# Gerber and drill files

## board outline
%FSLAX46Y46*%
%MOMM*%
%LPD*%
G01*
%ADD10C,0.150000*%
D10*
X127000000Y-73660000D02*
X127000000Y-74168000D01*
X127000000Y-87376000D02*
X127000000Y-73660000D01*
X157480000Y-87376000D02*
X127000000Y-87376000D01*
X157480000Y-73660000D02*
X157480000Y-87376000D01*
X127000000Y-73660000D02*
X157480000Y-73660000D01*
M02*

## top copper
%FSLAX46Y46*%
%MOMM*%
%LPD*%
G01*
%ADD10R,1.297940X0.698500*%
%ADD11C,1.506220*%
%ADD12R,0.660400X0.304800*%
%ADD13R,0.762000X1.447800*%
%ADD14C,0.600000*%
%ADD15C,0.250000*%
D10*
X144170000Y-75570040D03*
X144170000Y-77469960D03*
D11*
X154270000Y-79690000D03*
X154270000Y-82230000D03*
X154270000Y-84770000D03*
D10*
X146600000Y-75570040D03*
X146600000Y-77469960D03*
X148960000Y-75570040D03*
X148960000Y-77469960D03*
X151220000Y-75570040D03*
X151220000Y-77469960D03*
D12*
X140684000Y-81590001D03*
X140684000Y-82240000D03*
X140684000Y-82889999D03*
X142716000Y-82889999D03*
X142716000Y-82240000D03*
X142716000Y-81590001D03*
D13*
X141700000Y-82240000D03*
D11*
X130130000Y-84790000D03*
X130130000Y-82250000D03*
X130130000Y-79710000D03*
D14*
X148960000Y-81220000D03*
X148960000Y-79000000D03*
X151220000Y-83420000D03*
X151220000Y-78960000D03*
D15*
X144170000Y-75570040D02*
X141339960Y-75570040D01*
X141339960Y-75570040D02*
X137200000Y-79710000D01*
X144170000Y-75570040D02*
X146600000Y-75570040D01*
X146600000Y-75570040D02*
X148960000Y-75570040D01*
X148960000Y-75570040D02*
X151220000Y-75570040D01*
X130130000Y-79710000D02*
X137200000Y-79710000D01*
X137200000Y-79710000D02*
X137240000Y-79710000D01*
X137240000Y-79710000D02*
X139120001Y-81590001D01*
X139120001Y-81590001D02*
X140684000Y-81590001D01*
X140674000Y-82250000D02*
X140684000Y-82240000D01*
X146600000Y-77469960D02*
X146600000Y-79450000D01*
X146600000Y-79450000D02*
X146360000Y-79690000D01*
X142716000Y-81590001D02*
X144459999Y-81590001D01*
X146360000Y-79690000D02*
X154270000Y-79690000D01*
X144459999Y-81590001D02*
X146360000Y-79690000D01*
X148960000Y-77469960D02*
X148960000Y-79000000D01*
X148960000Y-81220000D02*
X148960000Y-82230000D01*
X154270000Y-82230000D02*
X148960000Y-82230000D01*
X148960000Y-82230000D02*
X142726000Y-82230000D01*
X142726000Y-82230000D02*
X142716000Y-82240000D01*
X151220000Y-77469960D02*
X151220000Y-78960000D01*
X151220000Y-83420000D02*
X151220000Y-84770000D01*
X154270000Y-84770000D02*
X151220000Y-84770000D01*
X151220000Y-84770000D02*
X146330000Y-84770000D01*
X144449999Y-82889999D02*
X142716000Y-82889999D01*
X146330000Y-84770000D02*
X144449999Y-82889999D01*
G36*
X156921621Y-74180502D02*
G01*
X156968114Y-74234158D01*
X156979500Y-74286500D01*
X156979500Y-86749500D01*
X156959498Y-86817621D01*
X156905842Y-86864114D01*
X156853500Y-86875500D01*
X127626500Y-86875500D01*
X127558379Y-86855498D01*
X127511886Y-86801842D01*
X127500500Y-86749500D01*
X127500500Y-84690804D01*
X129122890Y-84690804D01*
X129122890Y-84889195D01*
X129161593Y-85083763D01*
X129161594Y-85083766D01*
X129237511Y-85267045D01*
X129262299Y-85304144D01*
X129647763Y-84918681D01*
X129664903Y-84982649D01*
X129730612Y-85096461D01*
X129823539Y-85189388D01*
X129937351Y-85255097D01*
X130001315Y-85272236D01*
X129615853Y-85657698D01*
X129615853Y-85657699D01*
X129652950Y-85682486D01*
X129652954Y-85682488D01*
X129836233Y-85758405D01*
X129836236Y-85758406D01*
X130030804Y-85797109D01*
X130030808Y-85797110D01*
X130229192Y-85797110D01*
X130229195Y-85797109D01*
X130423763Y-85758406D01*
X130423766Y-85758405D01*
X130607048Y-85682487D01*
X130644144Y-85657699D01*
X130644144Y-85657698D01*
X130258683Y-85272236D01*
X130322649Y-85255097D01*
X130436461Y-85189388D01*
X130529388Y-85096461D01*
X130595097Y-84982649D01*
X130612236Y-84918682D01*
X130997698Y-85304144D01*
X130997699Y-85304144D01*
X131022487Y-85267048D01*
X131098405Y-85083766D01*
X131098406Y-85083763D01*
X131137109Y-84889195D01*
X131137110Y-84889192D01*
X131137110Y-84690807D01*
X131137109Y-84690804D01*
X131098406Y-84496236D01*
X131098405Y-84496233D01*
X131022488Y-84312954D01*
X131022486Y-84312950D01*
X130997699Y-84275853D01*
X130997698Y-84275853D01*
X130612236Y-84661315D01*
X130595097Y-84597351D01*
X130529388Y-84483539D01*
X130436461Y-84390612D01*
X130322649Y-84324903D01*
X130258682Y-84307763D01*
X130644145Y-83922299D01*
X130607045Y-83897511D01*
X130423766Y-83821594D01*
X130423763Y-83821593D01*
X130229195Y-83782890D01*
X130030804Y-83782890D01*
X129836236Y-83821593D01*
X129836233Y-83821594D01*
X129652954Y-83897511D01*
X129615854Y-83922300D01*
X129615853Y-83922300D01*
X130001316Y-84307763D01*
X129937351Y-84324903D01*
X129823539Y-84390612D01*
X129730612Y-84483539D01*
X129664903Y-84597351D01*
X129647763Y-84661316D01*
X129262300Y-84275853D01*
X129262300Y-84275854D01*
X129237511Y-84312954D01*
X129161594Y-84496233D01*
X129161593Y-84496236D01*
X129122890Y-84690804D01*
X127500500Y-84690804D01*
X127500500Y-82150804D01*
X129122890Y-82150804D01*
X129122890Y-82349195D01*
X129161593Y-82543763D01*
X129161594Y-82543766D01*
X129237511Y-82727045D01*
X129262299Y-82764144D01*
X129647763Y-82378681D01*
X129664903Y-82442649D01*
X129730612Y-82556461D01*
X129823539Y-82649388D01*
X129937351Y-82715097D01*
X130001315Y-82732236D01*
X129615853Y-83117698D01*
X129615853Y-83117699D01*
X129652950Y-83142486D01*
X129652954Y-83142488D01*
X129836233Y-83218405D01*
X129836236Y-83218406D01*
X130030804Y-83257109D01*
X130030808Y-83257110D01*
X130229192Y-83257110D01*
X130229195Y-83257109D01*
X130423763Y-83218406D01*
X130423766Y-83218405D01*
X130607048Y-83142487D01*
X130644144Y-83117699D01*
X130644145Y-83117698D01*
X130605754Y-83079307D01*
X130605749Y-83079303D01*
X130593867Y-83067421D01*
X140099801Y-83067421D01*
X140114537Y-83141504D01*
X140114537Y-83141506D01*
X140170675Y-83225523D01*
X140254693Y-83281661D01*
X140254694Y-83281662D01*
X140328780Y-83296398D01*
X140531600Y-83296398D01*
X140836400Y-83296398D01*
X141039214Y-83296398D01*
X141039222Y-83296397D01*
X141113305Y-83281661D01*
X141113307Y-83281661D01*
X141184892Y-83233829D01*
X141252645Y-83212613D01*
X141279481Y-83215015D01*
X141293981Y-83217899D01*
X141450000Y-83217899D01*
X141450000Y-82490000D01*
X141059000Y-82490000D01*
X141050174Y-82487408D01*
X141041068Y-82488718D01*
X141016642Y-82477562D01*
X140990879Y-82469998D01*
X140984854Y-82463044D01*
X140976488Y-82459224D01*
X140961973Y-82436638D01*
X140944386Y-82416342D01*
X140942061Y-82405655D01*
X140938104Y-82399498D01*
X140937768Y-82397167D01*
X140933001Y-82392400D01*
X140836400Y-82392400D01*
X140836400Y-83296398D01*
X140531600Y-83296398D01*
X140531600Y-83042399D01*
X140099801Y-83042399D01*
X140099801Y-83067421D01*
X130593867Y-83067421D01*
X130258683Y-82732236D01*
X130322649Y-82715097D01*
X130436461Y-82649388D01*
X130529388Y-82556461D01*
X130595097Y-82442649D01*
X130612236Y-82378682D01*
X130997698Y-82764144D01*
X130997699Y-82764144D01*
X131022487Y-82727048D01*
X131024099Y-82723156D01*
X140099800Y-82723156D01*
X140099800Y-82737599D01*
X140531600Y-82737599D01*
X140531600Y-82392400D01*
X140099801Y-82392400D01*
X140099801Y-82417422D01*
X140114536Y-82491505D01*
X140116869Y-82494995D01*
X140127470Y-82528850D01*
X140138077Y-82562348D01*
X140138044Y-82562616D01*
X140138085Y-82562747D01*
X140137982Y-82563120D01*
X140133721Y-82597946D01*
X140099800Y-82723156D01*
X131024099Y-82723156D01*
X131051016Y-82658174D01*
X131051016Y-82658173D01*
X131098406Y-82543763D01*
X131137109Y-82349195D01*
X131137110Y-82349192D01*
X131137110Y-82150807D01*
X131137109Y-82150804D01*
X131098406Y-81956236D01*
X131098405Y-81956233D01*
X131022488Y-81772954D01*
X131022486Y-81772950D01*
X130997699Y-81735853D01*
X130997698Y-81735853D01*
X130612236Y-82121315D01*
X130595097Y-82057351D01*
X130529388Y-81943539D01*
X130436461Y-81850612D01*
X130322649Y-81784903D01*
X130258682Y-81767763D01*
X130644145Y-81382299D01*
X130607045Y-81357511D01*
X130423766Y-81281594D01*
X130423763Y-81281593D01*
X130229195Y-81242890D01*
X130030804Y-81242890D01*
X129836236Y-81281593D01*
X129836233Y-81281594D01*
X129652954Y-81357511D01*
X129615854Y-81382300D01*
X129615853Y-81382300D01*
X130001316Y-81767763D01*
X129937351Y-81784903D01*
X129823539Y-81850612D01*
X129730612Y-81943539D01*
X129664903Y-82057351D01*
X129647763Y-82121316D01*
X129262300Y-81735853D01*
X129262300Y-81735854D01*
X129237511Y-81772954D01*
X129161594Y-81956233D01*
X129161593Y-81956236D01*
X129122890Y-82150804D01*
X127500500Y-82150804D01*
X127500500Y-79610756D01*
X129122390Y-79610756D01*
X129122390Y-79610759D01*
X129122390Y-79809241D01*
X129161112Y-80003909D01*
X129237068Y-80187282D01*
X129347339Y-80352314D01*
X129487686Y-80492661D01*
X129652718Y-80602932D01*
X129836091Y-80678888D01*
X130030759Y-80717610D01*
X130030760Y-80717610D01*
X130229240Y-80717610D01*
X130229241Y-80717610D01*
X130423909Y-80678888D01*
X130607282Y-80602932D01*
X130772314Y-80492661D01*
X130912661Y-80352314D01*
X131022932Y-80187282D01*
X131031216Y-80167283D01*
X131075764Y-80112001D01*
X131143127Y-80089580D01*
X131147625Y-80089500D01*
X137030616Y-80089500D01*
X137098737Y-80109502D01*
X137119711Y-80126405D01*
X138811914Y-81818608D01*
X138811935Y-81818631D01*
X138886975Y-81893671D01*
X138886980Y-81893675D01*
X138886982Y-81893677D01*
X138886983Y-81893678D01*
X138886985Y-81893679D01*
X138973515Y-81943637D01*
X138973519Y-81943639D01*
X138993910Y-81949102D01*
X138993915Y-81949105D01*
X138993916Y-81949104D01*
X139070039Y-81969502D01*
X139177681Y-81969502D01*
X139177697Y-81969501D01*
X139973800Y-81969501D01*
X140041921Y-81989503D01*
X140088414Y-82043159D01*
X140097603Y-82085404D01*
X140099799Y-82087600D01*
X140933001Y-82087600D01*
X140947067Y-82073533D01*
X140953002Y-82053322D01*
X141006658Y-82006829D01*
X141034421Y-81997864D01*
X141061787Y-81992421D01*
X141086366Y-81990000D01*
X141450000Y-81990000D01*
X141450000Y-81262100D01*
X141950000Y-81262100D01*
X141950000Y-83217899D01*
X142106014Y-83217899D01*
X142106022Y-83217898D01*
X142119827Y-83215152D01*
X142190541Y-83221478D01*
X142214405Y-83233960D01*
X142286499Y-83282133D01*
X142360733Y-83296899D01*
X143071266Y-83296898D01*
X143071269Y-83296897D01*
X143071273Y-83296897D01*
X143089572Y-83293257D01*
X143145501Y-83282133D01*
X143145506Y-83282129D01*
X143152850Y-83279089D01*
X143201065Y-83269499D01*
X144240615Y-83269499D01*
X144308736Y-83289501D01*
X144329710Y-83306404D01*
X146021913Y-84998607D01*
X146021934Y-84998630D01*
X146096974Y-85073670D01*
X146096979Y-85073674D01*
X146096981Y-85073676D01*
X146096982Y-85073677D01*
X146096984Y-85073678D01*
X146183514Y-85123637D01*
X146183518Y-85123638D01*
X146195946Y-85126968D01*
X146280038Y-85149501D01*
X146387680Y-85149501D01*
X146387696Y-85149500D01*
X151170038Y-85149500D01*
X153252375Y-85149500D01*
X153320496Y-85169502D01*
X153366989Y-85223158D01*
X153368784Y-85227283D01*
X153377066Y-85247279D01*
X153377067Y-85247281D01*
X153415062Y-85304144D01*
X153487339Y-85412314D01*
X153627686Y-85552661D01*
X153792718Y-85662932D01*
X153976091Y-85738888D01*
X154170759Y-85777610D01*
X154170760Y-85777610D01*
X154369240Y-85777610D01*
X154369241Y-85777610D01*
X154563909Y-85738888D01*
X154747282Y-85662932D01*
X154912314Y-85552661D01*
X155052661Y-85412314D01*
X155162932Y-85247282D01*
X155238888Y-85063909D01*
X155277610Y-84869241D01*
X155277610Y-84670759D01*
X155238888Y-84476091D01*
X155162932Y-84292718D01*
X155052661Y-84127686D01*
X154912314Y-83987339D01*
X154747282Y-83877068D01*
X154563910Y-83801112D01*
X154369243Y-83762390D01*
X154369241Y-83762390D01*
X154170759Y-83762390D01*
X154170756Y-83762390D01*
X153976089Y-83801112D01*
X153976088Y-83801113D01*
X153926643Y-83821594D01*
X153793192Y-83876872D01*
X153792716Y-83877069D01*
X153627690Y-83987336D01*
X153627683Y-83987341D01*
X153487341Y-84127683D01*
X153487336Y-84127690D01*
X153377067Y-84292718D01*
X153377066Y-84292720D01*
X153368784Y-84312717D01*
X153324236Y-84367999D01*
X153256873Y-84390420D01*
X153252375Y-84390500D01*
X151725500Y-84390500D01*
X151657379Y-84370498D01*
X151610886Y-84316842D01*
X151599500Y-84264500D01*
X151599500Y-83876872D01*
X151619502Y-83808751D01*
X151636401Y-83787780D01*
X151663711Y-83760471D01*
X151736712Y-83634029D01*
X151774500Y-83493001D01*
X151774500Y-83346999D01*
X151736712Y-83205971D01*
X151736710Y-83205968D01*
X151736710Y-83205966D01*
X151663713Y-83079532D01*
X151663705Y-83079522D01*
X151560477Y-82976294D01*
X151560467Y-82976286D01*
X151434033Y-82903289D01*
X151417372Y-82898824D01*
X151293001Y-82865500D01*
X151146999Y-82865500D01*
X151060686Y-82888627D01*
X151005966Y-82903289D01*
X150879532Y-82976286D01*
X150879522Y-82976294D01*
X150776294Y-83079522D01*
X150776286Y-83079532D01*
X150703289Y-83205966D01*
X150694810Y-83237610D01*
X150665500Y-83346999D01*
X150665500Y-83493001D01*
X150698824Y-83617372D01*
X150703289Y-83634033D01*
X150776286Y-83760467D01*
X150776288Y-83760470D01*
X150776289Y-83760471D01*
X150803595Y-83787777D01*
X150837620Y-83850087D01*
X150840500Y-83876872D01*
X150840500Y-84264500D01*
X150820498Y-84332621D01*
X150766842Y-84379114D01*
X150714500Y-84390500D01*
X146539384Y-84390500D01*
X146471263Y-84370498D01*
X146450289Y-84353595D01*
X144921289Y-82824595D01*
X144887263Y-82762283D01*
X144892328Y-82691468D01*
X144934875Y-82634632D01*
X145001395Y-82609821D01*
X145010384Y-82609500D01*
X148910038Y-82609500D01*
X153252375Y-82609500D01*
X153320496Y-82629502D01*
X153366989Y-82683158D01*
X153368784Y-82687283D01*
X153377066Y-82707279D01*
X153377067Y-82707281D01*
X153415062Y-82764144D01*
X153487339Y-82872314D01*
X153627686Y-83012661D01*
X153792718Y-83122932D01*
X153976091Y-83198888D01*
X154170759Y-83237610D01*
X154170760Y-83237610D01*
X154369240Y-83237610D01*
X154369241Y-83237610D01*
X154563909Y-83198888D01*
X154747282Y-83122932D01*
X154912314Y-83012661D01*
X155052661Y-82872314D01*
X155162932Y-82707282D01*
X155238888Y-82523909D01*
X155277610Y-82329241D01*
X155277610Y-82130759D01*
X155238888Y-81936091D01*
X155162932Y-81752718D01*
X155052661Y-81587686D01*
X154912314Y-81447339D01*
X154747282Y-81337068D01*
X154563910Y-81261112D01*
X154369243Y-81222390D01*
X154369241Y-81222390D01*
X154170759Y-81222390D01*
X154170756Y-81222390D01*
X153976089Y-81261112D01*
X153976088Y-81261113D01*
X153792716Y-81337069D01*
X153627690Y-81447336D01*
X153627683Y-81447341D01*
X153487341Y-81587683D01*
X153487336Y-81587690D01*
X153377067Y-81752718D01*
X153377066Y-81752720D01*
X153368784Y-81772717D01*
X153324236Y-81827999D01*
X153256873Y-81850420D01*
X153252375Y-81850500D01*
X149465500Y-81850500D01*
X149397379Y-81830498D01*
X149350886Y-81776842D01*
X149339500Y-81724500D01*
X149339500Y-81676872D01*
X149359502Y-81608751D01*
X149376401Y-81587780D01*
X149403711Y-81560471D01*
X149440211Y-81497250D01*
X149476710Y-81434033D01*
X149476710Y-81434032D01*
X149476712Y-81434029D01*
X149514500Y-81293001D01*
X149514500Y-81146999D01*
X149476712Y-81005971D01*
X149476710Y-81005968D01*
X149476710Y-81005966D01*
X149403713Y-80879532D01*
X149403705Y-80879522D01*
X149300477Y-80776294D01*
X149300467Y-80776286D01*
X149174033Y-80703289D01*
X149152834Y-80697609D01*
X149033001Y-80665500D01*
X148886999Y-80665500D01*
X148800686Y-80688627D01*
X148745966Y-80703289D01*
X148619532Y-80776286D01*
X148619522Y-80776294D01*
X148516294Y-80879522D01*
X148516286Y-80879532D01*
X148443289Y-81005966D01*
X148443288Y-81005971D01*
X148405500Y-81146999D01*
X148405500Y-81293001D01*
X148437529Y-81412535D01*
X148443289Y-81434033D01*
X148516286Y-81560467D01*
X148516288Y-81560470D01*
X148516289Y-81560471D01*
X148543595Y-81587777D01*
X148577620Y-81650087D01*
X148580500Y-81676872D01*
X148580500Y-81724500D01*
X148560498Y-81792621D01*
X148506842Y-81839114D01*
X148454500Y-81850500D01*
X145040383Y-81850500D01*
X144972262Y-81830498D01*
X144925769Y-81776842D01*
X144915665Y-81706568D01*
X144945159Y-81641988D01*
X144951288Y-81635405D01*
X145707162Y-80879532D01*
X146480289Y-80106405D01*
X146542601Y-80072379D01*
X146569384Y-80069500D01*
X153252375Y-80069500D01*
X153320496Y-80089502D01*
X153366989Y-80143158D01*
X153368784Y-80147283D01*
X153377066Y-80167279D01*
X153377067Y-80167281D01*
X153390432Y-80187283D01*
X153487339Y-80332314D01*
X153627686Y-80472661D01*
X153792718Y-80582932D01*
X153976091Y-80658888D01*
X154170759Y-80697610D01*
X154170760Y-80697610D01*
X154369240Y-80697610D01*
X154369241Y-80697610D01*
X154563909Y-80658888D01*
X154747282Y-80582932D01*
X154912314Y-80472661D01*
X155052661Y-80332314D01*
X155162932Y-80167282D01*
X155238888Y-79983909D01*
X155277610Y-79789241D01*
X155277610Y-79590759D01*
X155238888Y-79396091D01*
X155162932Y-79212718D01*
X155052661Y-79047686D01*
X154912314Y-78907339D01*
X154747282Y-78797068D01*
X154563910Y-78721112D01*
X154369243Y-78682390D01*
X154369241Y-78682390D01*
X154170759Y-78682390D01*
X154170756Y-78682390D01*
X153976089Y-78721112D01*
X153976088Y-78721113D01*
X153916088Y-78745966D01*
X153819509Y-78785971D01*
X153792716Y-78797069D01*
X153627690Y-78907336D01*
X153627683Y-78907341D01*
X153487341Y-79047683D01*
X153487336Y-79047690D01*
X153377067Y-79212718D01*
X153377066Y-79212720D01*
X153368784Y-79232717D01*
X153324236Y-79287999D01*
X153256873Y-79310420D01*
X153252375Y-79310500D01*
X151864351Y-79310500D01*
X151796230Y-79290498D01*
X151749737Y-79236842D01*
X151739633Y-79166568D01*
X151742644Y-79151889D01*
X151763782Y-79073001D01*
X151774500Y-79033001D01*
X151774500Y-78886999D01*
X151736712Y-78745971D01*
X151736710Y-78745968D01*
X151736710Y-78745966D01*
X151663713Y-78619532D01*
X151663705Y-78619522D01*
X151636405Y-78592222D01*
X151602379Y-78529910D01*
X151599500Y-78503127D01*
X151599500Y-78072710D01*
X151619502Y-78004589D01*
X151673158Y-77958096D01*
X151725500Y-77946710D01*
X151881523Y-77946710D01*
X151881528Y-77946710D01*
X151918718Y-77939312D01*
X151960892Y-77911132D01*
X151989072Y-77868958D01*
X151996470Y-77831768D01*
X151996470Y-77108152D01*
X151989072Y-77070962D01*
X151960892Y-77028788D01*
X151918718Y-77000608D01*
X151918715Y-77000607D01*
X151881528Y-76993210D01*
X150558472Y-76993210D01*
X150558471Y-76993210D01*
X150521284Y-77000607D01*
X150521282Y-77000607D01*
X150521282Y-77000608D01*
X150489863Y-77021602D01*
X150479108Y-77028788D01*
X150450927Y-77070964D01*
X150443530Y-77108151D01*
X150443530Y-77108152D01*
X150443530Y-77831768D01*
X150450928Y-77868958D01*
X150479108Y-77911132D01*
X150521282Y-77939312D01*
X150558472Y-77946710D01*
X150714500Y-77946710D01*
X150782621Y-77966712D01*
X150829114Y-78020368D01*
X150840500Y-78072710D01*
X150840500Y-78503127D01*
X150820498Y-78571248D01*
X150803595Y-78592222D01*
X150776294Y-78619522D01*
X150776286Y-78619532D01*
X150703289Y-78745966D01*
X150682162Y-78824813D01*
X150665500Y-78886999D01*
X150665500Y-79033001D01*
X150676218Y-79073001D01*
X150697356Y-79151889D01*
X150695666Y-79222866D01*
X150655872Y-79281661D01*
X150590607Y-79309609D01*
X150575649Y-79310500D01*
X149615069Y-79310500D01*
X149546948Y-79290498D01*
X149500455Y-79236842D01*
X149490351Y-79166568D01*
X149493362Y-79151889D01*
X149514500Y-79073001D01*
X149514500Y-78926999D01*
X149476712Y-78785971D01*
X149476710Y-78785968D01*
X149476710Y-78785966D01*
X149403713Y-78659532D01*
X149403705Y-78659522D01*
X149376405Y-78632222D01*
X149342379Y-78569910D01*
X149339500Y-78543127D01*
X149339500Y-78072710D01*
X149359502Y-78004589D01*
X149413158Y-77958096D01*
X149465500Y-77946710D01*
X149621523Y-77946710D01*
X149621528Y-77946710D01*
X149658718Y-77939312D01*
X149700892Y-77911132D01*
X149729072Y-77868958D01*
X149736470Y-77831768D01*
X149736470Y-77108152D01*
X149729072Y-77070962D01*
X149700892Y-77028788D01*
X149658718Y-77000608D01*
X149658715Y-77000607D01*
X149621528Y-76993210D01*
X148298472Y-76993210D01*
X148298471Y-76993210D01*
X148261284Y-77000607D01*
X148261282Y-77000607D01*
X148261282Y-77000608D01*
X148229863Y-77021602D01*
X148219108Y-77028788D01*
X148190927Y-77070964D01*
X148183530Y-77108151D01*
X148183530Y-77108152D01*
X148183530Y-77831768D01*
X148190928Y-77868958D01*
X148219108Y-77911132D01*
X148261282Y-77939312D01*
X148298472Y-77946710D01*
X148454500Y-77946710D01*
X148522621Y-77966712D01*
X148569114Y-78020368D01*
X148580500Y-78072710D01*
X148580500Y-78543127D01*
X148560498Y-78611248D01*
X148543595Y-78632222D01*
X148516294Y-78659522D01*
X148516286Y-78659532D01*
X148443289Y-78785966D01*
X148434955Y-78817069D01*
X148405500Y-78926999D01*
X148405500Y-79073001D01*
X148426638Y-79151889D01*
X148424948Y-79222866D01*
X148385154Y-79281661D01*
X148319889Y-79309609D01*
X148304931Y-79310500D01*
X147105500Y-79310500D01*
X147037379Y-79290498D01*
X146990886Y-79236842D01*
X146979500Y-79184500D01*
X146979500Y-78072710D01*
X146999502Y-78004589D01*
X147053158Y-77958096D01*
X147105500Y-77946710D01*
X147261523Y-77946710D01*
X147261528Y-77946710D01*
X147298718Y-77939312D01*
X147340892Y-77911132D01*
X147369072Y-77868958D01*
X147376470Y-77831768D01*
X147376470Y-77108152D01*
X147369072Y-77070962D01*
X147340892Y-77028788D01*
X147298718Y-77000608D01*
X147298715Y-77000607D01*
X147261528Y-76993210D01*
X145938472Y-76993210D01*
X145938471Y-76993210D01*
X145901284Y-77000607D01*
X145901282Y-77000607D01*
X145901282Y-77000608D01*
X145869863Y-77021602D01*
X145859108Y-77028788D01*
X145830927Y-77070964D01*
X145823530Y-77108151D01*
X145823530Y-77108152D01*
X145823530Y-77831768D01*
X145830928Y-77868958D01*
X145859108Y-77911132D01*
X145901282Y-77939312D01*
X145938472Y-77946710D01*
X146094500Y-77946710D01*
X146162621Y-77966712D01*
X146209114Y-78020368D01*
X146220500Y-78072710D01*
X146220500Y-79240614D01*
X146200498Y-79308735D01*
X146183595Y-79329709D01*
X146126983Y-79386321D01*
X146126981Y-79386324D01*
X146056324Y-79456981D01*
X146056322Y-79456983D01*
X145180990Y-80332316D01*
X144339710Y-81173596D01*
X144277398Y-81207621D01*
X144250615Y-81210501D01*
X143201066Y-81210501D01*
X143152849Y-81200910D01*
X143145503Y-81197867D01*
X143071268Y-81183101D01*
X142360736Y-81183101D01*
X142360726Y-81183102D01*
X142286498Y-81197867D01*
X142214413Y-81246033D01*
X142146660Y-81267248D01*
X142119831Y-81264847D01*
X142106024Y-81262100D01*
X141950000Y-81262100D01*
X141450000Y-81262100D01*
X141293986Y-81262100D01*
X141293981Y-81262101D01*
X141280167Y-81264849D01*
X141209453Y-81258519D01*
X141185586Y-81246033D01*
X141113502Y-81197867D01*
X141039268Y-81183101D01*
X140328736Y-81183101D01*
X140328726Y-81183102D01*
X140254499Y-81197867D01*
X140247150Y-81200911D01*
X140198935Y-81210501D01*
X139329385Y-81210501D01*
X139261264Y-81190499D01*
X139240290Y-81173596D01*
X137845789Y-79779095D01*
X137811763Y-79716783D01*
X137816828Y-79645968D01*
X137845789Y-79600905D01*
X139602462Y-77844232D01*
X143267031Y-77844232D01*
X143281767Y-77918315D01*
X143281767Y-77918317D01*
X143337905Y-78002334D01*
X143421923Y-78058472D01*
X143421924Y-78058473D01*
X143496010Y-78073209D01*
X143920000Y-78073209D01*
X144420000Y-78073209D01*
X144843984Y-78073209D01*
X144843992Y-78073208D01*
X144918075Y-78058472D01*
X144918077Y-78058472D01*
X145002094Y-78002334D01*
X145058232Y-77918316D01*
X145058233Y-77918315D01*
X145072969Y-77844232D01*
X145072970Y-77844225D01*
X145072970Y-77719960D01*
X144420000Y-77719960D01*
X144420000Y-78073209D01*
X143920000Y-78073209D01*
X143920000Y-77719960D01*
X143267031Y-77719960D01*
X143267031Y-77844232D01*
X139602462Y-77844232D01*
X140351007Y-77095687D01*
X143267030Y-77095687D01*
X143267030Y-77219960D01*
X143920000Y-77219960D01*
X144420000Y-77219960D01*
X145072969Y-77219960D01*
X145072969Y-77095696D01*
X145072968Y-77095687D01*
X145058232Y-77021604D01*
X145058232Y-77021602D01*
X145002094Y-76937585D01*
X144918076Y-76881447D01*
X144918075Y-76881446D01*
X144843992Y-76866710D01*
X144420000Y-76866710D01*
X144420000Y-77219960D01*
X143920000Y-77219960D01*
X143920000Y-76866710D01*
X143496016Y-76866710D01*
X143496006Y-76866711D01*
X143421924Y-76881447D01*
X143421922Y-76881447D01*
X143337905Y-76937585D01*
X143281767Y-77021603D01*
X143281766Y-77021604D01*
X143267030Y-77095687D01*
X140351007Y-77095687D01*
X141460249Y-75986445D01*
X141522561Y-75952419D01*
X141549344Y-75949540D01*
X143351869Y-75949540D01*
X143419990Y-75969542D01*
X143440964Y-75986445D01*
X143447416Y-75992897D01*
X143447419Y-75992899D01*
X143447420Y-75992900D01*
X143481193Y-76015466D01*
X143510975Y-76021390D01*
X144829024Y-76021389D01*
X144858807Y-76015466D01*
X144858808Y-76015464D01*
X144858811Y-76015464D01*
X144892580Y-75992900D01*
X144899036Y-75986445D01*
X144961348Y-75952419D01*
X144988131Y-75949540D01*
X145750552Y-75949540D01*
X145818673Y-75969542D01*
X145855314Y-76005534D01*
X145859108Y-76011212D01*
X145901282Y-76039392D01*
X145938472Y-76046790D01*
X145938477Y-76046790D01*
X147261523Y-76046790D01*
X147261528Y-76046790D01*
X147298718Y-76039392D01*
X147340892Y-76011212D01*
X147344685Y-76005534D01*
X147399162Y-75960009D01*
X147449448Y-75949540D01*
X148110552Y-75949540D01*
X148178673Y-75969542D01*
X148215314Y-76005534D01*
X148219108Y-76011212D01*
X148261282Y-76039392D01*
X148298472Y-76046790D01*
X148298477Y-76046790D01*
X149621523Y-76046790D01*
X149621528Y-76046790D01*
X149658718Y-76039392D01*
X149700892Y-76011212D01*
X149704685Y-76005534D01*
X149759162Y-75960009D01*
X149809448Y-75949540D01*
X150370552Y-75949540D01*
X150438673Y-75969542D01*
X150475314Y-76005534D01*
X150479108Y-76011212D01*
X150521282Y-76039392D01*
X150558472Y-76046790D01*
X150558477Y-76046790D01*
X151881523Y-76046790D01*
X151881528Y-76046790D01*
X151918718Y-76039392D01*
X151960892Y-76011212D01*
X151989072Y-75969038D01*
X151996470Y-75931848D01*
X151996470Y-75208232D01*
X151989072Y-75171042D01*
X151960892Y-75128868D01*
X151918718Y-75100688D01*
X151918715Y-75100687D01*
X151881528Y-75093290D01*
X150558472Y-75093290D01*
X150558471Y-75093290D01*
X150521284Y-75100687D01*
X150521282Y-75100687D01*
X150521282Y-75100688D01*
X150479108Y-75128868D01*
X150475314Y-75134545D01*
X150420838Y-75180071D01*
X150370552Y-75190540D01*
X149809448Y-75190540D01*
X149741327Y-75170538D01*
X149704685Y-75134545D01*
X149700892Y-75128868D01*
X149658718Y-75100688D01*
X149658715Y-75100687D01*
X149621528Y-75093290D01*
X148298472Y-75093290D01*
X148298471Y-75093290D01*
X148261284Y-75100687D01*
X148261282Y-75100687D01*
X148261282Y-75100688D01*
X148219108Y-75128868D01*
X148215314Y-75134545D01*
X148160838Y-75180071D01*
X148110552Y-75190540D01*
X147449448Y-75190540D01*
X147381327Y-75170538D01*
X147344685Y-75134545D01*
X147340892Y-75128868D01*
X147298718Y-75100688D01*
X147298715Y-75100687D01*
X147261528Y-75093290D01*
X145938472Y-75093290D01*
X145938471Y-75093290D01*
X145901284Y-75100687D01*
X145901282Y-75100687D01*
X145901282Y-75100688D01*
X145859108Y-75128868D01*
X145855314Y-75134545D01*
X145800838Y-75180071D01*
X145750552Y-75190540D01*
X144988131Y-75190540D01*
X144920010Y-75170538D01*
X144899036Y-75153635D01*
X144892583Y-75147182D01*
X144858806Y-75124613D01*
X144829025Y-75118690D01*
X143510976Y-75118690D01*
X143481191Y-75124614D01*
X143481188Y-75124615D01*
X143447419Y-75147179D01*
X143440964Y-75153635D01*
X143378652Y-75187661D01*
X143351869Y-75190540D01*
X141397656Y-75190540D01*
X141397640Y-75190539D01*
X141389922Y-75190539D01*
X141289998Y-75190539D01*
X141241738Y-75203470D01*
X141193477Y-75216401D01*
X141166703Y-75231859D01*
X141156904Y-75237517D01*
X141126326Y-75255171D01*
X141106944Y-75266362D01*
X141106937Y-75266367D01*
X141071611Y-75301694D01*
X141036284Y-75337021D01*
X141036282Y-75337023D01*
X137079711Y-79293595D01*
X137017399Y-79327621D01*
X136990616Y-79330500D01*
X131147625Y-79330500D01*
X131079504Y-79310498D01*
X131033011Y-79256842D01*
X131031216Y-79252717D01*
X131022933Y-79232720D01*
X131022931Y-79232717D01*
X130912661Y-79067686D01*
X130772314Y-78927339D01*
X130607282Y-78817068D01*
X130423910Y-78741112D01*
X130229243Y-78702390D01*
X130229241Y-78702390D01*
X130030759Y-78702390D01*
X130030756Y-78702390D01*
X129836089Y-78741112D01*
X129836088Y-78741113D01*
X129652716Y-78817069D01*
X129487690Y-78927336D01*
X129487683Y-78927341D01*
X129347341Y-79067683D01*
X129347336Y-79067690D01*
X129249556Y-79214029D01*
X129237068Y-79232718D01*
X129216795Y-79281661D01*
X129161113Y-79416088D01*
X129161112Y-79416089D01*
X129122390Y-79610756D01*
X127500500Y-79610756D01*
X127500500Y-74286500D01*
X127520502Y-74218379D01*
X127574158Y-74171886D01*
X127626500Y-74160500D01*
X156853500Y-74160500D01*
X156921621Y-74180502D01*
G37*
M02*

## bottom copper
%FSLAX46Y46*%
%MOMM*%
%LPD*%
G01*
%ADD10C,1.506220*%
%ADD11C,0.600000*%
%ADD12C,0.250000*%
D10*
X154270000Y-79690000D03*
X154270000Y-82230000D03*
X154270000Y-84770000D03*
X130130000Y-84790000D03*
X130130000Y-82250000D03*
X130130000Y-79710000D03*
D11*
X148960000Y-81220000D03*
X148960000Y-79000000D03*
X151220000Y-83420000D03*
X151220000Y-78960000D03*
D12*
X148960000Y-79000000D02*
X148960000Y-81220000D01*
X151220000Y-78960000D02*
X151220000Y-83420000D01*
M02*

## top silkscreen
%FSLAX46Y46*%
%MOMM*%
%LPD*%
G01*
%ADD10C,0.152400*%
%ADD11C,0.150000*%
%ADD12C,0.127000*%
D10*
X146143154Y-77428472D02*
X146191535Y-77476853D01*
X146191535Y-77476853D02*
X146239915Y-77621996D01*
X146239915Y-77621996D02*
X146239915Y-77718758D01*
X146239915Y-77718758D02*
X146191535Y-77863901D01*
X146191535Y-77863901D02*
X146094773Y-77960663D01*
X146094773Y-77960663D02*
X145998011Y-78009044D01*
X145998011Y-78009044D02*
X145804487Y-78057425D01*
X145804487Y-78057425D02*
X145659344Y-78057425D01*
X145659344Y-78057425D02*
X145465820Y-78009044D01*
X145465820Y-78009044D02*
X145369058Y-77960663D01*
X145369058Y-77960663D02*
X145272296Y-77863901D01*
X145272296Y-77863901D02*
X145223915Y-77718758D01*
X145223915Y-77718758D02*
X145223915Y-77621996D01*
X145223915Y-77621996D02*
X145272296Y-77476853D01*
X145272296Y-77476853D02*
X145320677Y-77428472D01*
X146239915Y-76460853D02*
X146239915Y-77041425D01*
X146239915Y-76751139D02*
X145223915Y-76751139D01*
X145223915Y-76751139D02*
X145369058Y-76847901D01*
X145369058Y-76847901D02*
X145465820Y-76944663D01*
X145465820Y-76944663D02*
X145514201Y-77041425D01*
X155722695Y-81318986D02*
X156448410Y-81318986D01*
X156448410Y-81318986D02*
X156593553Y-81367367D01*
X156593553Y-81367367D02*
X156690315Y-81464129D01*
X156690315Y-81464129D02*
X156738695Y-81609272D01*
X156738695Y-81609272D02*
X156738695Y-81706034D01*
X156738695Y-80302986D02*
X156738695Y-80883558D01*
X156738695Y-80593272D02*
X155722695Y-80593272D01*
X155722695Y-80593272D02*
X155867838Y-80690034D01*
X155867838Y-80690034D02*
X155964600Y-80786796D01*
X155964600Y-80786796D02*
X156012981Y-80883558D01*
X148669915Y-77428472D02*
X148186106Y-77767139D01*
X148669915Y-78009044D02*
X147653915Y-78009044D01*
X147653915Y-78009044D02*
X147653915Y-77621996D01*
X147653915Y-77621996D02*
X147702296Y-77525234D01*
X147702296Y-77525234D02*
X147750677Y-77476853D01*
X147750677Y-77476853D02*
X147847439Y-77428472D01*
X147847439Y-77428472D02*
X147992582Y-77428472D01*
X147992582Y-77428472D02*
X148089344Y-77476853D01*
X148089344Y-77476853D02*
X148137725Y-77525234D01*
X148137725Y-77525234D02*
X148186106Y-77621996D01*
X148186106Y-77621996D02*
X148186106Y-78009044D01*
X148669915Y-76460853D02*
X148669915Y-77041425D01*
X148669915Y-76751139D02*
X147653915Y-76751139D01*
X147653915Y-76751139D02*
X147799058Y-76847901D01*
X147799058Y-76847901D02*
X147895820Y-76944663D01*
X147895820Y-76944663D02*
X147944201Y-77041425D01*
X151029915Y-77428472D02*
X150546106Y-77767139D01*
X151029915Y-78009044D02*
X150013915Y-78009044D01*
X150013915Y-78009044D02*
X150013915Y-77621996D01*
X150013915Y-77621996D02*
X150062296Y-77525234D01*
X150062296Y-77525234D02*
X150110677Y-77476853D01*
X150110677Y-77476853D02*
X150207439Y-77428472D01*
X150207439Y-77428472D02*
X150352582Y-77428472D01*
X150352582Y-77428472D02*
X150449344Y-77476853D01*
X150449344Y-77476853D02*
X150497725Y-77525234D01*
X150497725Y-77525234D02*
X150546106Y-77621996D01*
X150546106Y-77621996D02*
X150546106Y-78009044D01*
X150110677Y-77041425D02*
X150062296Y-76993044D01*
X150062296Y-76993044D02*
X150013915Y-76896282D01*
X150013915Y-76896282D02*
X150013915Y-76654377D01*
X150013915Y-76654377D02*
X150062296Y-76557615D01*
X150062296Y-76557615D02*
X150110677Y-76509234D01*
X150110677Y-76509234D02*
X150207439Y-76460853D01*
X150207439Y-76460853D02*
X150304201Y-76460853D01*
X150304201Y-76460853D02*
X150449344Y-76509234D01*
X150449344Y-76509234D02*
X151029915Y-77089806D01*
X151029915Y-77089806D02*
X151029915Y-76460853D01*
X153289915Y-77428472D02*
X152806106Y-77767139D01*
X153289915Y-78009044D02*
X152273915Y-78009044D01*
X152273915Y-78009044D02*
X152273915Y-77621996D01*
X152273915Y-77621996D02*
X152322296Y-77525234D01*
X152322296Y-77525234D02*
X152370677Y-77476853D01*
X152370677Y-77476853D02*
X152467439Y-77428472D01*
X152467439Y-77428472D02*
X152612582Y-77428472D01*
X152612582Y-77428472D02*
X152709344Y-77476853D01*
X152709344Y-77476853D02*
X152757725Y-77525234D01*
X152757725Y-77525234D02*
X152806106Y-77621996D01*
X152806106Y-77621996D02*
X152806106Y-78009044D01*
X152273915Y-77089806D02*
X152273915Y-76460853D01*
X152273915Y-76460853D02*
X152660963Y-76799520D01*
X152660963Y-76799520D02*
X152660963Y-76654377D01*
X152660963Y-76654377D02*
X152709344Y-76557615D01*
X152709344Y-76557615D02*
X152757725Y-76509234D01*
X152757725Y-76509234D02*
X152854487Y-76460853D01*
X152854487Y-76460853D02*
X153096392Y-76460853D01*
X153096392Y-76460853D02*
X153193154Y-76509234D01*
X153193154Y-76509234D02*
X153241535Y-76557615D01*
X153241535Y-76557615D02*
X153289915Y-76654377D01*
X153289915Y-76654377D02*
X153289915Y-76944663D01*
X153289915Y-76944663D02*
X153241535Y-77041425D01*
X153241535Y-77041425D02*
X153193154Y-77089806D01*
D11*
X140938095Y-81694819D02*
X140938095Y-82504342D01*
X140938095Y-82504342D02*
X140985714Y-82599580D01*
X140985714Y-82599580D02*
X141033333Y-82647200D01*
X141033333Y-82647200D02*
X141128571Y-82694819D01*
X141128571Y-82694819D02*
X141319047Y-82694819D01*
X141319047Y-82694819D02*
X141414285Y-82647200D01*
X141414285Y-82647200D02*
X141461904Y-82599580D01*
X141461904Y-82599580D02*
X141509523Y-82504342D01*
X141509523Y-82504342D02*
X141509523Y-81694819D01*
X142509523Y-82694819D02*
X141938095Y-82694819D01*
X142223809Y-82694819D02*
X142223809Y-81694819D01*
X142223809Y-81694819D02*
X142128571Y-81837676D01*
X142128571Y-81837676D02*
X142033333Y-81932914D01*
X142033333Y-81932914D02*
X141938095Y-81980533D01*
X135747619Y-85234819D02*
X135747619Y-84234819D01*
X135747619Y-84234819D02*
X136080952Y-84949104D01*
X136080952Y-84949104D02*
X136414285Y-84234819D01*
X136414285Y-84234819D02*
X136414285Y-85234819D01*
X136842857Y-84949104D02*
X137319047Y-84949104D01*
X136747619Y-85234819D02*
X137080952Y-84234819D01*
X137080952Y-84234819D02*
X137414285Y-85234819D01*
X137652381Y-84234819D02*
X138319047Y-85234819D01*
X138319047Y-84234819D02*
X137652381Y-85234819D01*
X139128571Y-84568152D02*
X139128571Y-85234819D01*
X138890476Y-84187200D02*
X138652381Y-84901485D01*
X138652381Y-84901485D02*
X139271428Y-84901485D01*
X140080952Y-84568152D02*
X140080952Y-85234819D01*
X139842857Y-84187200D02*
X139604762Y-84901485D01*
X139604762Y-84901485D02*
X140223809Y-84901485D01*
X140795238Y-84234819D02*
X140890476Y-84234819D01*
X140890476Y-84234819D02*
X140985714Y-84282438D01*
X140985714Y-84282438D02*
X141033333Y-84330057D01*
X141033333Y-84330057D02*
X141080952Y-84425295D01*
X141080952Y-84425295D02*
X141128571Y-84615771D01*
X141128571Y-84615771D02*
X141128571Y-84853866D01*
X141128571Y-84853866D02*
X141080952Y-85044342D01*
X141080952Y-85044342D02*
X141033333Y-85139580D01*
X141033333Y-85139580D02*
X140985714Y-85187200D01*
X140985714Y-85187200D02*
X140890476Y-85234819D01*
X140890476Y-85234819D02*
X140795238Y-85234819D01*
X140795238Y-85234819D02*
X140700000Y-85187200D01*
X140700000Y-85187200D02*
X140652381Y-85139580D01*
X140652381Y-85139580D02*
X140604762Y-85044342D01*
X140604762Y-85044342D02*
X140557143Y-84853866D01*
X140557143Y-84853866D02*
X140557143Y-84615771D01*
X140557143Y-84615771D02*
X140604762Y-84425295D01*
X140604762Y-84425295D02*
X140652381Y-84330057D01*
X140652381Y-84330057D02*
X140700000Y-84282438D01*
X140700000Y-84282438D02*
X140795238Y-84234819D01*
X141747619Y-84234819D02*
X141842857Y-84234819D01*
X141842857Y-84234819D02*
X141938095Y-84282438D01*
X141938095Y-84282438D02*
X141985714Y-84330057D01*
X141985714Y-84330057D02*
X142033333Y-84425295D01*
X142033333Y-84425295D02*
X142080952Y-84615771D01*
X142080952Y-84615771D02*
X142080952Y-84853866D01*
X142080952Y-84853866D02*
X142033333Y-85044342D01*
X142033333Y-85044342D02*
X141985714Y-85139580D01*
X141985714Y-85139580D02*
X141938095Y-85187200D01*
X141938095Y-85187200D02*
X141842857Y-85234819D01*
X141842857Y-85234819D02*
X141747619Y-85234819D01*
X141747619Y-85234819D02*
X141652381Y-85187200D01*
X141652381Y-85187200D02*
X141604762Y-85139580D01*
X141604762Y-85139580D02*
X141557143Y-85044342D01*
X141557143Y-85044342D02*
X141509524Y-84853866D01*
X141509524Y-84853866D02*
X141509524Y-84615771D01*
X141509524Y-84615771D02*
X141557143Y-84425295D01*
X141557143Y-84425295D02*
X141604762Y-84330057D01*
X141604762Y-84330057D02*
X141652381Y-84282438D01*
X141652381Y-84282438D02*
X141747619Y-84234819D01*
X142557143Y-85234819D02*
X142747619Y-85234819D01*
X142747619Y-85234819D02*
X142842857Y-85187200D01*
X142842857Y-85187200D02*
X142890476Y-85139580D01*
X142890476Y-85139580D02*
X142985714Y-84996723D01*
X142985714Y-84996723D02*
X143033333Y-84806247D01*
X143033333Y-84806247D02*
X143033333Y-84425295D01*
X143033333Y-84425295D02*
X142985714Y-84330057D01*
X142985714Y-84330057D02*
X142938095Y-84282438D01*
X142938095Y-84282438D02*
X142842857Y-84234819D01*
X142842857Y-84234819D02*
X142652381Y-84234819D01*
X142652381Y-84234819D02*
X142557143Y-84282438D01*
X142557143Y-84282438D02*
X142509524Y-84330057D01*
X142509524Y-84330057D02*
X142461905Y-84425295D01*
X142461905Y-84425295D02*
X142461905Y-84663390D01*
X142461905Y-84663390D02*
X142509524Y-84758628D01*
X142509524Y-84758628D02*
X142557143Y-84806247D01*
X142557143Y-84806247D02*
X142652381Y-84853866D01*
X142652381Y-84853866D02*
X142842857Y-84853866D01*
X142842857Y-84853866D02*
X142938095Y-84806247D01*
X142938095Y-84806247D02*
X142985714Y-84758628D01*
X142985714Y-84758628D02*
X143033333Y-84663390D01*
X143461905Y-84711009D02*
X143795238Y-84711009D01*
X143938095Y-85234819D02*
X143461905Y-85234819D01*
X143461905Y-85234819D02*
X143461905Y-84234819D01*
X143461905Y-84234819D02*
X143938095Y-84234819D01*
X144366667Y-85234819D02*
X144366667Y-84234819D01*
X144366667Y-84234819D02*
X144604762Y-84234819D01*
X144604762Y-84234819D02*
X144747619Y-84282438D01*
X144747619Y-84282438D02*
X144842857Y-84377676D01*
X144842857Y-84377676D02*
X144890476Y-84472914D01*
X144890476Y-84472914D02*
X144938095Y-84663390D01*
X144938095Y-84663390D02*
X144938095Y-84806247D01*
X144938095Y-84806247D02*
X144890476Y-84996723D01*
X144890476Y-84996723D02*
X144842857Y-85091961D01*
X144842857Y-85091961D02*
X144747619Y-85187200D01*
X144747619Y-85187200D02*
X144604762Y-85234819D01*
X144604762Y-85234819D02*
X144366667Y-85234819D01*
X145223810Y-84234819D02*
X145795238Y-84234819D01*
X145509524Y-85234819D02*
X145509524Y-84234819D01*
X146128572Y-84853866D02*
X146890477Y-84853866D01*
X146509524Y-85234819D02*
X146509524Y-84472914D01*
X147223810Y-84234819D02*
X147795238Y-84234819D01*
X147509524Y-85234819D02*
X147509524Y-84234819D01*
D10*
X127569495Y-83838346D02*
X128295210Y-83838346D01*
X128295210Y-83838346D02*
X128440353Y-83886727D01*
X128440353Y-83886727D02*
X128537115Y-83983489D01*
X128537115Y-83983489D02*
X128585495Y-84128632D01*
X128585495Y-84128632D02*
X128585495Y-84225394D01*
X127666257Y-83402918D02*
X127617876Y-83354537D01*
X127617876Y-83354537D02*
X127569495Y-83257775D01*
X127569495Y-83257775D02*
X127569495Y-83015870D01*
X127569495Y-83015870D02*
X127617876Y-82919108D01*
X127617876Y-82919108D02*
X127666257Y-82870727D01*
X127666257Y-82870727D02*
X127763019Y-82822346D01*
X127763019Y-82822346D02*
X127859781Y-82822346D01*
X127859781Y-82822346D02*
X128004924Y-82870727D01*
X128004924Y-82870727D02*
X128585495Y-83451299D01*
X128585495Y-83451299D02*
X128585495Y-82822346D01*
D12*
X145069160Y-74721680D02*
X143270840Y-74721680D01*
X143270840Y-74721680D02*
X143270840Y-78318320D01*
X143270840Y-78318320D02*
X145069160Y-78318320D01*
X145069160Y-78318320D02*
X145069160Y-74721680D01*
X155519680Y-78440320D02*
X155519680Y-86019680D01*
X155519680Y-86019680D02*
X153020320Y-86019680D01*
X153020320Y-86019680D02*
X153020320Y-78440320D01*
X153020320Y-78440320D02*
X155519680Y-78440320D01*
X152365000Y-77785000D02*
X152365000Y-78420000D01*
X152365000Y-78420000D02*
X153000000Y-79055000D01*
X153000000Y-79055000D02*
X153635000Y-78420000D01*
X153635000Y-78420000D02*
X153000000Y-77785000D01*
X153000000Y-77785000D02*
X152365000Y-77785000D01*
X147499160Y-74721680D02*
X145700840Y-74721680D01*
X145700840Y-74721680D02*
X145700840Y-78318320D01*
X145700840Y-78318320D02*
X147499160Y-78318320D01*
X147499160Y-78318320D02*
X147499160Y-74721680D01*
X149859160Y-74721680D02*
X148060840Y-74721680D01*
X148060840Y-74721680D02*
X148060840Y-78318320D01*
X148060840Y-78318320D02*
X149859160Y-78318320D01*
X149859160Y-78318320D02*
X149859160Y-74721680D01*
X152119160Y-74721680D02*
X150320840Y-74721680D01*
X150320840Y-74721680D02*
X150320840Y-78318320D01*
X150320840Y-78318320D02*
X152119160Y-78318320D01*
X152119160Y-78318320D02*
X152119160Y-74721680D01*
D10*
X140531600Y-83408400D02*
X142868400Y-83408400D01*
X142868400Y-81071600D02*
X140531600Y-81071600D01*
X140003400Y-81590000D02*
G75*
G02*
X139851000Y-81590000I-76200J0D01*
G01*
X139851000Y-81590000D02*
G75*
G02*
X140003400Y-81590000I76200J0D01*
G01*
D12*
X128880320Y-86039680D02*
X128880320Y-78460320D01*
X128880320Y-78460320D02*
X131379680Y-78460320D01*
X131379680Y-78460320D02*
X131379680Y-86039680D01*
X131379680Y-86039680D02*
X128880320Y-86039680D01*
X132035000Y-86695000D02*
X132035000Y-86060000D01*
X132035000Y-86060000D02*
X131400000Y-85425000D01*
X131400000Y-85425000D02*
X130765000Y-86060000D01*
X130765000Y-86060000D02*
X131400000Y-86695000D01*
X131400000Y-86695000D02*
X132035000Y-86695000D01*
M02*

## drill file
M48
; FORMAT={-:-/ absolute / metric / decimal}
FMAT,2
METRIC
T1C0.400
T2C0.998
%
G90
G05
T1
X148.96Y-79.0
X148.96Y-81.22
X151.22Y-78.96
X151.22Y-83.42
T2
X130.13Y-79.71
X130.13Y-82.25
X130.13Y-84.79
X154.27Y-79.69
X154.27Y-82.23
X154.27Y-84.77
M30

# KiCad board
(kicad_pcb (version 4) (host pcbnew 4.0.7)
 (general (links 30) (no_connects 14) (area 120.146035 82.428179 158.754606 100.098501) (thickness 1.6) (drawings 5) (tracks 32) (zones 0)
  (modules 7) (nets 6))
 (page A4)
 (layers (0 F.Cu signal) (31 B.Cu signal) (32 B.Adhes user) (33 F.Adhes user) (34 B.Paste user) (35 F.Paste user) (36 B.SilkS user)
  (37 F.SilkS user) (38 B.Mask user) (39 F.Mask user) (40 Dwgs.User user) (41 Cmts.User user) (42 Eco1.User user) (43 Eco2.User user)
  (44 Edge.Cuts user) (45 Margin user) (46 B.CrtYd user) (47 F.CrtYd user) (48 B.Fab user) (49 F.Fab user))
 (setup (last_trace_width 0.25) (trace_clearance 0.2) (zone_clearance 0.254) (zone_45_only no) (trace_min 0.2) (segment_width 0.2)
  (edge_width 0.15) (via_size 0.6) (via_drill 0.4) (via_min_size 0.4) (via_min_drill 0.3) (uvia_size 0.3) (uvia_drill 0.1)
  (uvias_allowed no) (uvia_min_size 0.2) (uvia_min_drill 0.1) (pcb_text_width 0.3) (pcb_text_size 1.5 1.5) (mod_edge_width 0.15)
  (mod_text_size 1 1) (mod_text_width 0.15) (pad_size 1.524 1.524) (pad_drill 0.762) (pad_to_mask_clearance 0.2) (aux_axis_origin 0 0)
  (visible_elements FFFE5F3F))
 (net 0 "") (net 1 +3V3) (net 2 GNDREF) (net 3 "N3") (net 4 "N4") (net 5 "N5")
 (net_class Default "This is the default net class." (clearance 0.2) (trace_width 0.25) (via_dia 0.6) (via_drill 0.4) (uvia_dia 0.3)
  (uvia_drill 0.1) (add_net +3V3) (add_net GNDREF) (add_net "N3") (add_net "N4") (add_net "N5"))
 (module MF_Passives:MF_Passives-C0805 (layer F.Cu) (at 144.17 76.52 270) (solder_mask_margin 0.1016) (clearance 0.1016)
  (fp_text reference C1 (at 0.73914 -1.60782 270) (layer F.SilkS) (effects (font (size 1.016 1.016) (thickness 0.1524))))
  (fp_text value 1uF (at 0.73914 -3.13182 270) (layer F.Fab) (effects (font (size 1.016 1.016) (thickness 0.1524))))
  (fp_line (start -1.79832 -0.89916) (end -1.79832 0.89916) (layer F.SilkS) (width 0.127))
  (fp_line (start -1.79832 0.89916) (end 1.79832 0.89916) (layer F.SilkS) (width 0.127))
  (fp_line (start 1.79832 0.89916) (end 1.79832 -0.89916) (layer F.SilkS) (width 0.127))
  (fp_line (start 1.79832 -0.89916) (end -1.79832 -0.89916) (layer F.SilkS) (width 0.127))
  (pad 1 smd rect (at -0.94996 0 90) (size 0.6985 1.29794) (layers F.Cu F.Paste F.Mask) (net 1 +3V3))
  (pad 2 smd rect (at 0.94996 0 90) (size 0.6985 1.29794) (layers F.Cu F.Paste F.Mask) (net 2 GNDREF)))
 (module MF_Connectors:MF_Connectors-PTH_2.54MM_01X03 (layer F.Cu) (at 154.27 82.23 270)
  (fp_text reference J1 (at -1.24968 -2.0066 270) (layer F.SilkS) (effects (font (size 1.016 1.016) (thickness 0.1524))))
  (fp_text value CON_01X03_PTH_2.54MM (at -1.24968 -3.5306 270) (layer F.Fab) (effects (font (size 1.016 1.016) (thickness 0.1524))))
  (fp_line (start -3.78968 -1.24968) (end 3.78968 -1.24968) (layer F.SilkS) (width 0.127))
  (fp_line (start 3.78968 -1.24968) (end 3.78968 1.24968) (layer F.SilkS) (width 0.127))
  (fp_line (start 3.78968 1.24968) (end -3.78968 1.24968) (layer F.SilkS) (width 0.127))
  (fp_line (start -3.78968 1.24968) (end -3.78968 -1.24968) (layer F.SilkS) (width 0.127))
  (fp_line (start -4.445 1.905) (end -3.81 1.905) (layer F.SilkS) (width 0.127))
  (fp_line (start -3.81 1.905) (end -3.175 1.27) (layer F.SilkS) (width 0.127))
  (fp_line (start -3.175 1.27) (end -3.81 0.635) (layer F.SilkS) (width 0.127))
  (fp_line (start -3.81 0.635) (end -4.445 1.27) (layer F.SilkS) (width 0.127))
  (fp_line (start -4.445 1.27) (end -4.445 1.905) (layer F.SilkS) (width 0.127))
  (pad 1 thru_hole circle (at -2.54 0 270) (size 1.50622 1.50622) (drill 0.99822) (layers *.Cu *.Mask) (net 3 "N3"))
  (pad 2 thru_hole circle (at 0 0 270) (size 1.50622 1.50622) (drill 0.99822) (layers *.Cu *.Mask) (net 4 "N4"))
  (pad 3 thru_hole circle (at 2.54 0 270) (size 1.50622 1.50622) (drill 0.99822) (layers *.Cu *.Mask) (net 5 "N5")))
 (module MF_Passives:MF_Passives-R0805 (layer F.Cu) (at 146.6 76.52 270) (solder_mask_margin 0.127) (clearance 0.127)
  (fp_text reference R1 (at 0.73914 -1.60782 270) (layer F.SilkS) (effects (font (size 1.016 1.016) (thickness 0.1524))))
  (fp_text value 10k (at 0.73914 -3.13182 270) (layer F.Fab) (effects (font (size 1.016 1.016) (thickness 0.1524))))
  (fp_line (start -1.79832 -0.89916) (end -1.79832 0.89916) (layer F.SilkS) (width 0.127))
  (fp_line (start -1.79832 0.89916) (end 1.79832 0.89916) (layer F.SilkS) (width 0.127))
  (fp_line (start 1.79832 0.89916) (end 1.79832 -0.89916) (layer F.SilkS) (width 0.127))
  (fp_line (start 1.79832 -0.89916) (end -1.79832 -0.89916) (layer F.SilkS) (width 0.127))
  (pad 1 smd rect (at -0.94996 0 90) (size 0.6985 1.29794) (layers F.Cu F.Paste F.Mask) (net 1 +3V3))
  (pad 2 smd rect (at 0.94996 0 90) (size 0.6985 1.29794) (layers F.Cu F.Paste F.Mask) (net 3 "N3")))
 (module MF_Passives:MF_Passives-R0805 (layer F.Cu) (at 148.96 76.52 270) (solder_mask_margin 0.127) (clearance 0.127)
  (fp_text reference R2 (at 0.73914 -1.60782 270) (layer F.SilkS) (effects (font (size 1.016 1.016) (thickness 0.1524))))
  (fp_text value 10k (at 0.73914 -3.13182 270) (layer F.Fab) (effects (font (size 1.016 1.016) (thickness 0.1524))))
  (fp_line (start -1.79832 -0.89916) (end -1.79832 0.89916) (layer F.SilkS) (width 0.127))
  (fp_line (start -1.79832 0.89916) (end 1.79832 0.89916) (layer F.SilkS) (width 0.127))
  (fp_line (start 1.79832 0.89916) (end 1.79832 -0.89916) (layer F.SilkS) (width 0.127))
  (fp_line (start 1.79832 -0.89916) (end -1.79832 -0.89916) (layer F.SilkS) (width 0.127))
  (pad 1 smd rect (at -0.94996 0 90) (size 0.6985 1.29794) (layers F.Cu F.Paste F.Mask) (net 1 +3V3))
  (pad 2 smd rect (at 0.94996 0 90) (size 0.6985 1.29794) (layers F.Cu F.Paste F.Mask) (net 4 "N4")))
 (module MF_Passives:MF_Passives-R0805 (layer F.Cu) (at 151.22 76.52 270) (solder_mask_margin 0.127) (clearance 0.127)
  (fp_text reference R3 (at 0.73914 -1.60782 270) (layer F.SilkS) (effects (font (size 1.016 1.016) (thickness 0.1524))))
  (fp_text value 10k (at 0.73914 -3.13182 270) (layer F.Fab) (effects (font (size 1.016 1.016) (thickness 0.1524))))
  (fp_line (start -1.79832 -0.89916) (end -1.79832 0.89916) (layer F.SilkS) (width 0.127))
  (fp_line (start -1.79832 0.89916) (end 1.79832 0.89916) (layer F.SilkS) (width 0.127))
  (fp_line (start 1.79832 0.89916) (end 1.79832 -0.89916) (layer F.SilkS) (width 0.127))
  (fp_line (start 1.79832 -0.89916) (end -1.79832 -0.89916) (layer F.SilkS) (width 0.127))
  (pad 1 smd rect (at -0.94996 0 90) (size 0.6985 1.29794) (layers F.Cu F.Paste F.Mask) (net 1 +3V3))
  (pad 2 smd rect (at 0.94996 0 90) (size 0.6985 1.29794) (layers F.Cu F.Paste F.Mask) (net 5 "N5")))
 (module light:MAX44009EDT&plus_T (layer F.Cu) (at 141.7 82.24)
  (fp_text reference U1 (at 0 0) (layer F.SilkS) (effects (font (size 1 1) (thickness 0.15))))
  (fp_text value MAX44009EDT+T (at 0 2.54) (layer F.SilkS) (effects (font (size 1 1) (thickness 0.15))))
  (fp_line (start -1.1684 1.1684) (end 1.1684 1.1684) (layer F.SilkS) (width 0.1524))
  (fp_line (start 1.1684 -1.1684) (end -1.1684 -1.1684) (layer F.SilkS) (width 0.1524))
  (fp_circle (center -1.7728 -0.65) (end -1.6966 -0.65) (layer F.SilkS) (width 0.1524))
  (pad 1 smd rect (at -1.016 -0.649999) (size 0.6604 0.3048) (layers F.Cu) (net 1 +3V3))
  (pad 1 smd rect (at -1.016 -0.649999) (size 0.6604 0.3048) (layers F.Paste) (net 1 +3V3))
  (pad 1 smd rect (at -1.016 -0.649999) (size 0.6604 0.3048) (layers F.Mask) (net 1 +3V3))
  (pad 2 smd rect (at -1.016 0) (size 0.6604 0.3048) (layers F.Cu) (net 2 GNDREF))
  (pad 2 smd rect (at -1.016 0) (size 0.6604 0.3048) (layers F.Paste) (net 2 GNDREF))
  (pad 2 smd rect (at -1.016 0) (size 0.6604 0.3048) (layers F.Mask) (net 2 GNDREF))
  (pad 3 smd rect (at -1.016 0.649999) (size 0.6604 0.3048) (layers F.Cu) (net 2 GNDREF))
  (pad 3 smd rect (at -1.016 0.649999) (size 0.6604 0.3048) (layers F.Paste) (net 2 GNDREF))
  (pad 3 smd rect (at -1.016 0.649999) (size 0.6604 0.3048) (layers F.Mask) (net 2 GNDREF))
  (pad 4 smd rect (at 1.016 0.649999) (size 0.6604 0.3048) (layers F.Cu) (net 5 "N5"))
  (pad 4 smd rect (at 1.016 0.649999) (size 0.6604 0.3048) (layers F.Paste) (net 5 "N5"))
  (pad 4 smd rect (at 1.016 0.649999) (size 0.6604 0.3048) (layers F.Mask) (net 5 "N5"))
  (pad 5 smd rect (at 1.016 0) (size 0.6604 0.3048) (layers F.Cu) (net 4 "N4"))
  (pad 5 smd rect (at 1.016 0) (size 0.6604 0.3048) (layers F.Paste) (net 4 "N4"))
  (pad 5 smd rect (at 1.016 0) (size 0.6604 0.3048) (layers F.Mask) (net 4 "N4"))
  (pad 6 smd rect (at 1.016 -0.649999) (size 0.6604 0.3048) (layers F.Cu) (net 3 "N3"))
  (pad 6 smd rect (at 1.016 -0.649999) (size 0.6604 0.3048) (layers F.Paste) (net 3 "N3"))
  (pad 6 smd rect (at 1.016 -0.649999) (size 0.6604 0.3048) (layers F.Mask) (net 3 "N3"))
  (pad 7 smd rect (at 0 0) (size 0.762 1.4478) (layers F.Cu) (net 2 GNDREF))
  (pad 7 smd rect (at 0 0) (size 0.0254 0.0254) (layers F.Paste) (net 2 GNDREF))
  (pad 7 smd rect (at 0 0) (size 0.762 1.4478) (layers F.Mask) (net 2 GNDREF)))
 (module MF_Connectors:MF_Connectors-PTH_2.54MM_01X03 (layer F.Cu) (at 130.13 82.25 90)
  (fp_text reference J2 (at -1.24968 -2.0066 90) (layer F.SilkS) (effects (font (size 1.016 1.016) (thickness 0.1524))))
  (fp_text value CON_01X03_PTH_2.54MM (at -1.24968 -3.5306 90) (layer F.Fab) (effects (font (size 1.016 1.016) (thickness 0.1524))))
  (fp_line (start -3.78968 -1.24968) (end 3.78968 -1.24968) (layer F.SilkS) (width 0.127))
  (fp_line (start 3.78968 -1.24968) (end 3.78968 1.24968) (layer F.SilkS) (width 0.127))
  (fp_line (start 3.78968 1.24968) (end -3.78968 1.24968) (layer F.SilkS) (width 0.127))
  (fp_line (start -3.78968 1.24968) (end -3.78968 -1.24968) (layer F.SilkS) (width 0.127))
  (fp_line (start -4.445 1.905) (end -3.81 1.905) (layer F.SilkS) (width 0.127))
  (fp_line (start -3.81 1.905) (end -3.175 1.27) (layer F.SilkS) (width 0.127))
  (fp_line (start -3.175 1.27) (end -3.81 0.635) (layer F.SilkS) (width 0.127))
  (fp_line (start -3.81 0.635) (end -4.445 1.27) (layer F.SilkS) (width 0.127))
  (fp_line (start -4.445 1.27) (end -4.445 1.905) (layer F.SilkS) (width 0.127))
  (pad 1 thru_hole circle (at -2.54 0 90) (size 1.50622 1.50622) (drill 0.99822) (layers *.Cu *.Mask) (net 2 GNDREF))
  (pad 2 thru_hole circle (at 0 0 90) (size 1.50622 1.50622) (drill 0.99822) (layers *.Cu *.Mask) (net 2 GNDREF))
  (pad 3 thru_hole circle (at 2.54 0 90) (size 1.50622 1.50622) (drill 0.99822) (layers *.Cu *.Mask) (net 1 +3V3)))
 (gr_line (start 127 73.66) (end 127 74.168) (angle 90) (layer Edge.Cuts) (width 0.15))
 (gr_line (start 127 87.376) (end 127 73.66) (angle 90) (layer Edge.Cuts) (width 0.15))
 (gr_line (start 157.48 87.376) (end 127 87.376) (angle 90) (layer Edge.Cuts) (width 0.15))
 (gr_line (start 157.48 73.66) (end 157.48 87.376) (angle 90) (layer Edge.Cuts) (width 0.15))
 (gr_line (start 127 73.66) (end 157.48 73.66) (angle 90) (layer Edge.Cuts) (width 0.15))
 (segment (start 144.17 75.57004) (end 141.33996 75.57004) (width 0.25) (layer F.Cu) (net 1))
 (segment (start 141.33996 75.57004) (end 137.2 79.71) (width 0.25) (layer F.Cu) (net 1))
 (segment (start 144.17 75.57004) (end 146.6 75.57004) (width 0.25) (layer F.Cu) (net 1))
 (segment (start 146.6 75.57004) (end 148.96 75.57004) (width 0.25) (layer F.Cu) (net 1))
 (segment (start 148.96 75.57004) (end 151.22 75.57004) (width 0.25) (layer F.Cu) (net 1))
 (segment (start 130.13 79.71) (end 137.2 79.71) (width 0.25) (layer F.Cu) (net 1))
 (segment (start 137.2 79.71) (end 137.24 79.71) (width 0.25) (layer F.Cu) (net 1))
 (segment (start 137.24 79.71) (end 139.120001 81.590001) (width 0.25) (layer F.Cu) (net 1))
 (segment (start 139.120001 81.590001) (end 140.684 81.590001) (width 0.25) (layer F.Cu) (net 1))
 (segment (start 140.674 82.25) (end 140.684 82.24) (width 0.25) (layer F.Cu) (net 2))
 (segment (start 146.6 77.46996) (end 146.6 79.45) (width 0.25) (layer F.Cu) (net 3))
 (segment (start 146.6 79.45) (end 146.36 79.69) (width 0.25) (layer F.Cu) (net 3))
 (segment (start 142.716 81.590001) (end 144.459999 81.590001) (width 0.25) (layer F.Cu) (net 3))
 (segment (start 146.36 79.69) (end 154.27 79.69) (width 0.25) (layer F.Cu) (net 3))
 (segment (start 144.459999 81.590001) (end 146.36 79.69) (width 0.25) (layer F.Cu) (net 3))
 (segment (start 148.96 77.46996) (end 148.96 79) (width 0.25) (layer F.Cu) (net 4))
 (segment (start 148.96 81.22) (end 148.96 82.23) (width 0.25) (layer F.Cu) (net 4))
 (via (at 148.96 81.22) (size 0.6) (drill 0.4) (layers F.Cu B.Cu) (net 4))
 (segment (start 148.96 79) (end 148.96 81.22) (width 0.25) (layer B.Cu) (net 4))
 (via (at 148.96 79) (size 0.6) (drill 0.4) (layers F.Cu B.Cu) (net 4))
 (segment (start 154.27 82.23) (end 148.96 82.23) (width 0.25) (layer F.Cu) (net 4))
 (segment (start 148.96 82.23) (end 142.726 82.23) (width 0.25) (layer F.Cu) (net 4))
 (segment (start 142.726 82.23) (end 142.716 82.24) (width 0.25) (layer F.Cu) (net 4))
 (segment (start 151.22 77.46996) (end 151.22 78.96) (width 0.25) (layer F.Cu) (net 5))
 (segment (start 151.22 83.42) (end 151.22 84.77) (width 0.25) (layer F.Cu) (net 5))
 (via (at 151.22 83.42) (size 0.6) (drill 0.4) (layers F.Cu B.Cu) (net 5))
 (segment (start 151.22 78.96) (end 151.22 83.42) (width 0.25) (layer B.Cu) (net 5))
 (via (at 151.22 78.96) (size 0.6) (drill 0.4) (layers F.Cu B.Cu) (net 5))
 (segment (start 154.27 84.77) (end 151.22 84.77) (width 0.25) (layer F.Cu) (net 5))
 (segment (start 151.22 84.77) (end 146.33 84.77) (width 0.25) (layer F.Cu) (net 5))
 (segment (start 144.449999 82.889999) (end 142.716 82.889999) (width 0.25) (layer F.Cu) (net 5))
 (segment (start 146.33 84.77) (end 144.449999 82.889999) (width 0.25) (layer F.Cu) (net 5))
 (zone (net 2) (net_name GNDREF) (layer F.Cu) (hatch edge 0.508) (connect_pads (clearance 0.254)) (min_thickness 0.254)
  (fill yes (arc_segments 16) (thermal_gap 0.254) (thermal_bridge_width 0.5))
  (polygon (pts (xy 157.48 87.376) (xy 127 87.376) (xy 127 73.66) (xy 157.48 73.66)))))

